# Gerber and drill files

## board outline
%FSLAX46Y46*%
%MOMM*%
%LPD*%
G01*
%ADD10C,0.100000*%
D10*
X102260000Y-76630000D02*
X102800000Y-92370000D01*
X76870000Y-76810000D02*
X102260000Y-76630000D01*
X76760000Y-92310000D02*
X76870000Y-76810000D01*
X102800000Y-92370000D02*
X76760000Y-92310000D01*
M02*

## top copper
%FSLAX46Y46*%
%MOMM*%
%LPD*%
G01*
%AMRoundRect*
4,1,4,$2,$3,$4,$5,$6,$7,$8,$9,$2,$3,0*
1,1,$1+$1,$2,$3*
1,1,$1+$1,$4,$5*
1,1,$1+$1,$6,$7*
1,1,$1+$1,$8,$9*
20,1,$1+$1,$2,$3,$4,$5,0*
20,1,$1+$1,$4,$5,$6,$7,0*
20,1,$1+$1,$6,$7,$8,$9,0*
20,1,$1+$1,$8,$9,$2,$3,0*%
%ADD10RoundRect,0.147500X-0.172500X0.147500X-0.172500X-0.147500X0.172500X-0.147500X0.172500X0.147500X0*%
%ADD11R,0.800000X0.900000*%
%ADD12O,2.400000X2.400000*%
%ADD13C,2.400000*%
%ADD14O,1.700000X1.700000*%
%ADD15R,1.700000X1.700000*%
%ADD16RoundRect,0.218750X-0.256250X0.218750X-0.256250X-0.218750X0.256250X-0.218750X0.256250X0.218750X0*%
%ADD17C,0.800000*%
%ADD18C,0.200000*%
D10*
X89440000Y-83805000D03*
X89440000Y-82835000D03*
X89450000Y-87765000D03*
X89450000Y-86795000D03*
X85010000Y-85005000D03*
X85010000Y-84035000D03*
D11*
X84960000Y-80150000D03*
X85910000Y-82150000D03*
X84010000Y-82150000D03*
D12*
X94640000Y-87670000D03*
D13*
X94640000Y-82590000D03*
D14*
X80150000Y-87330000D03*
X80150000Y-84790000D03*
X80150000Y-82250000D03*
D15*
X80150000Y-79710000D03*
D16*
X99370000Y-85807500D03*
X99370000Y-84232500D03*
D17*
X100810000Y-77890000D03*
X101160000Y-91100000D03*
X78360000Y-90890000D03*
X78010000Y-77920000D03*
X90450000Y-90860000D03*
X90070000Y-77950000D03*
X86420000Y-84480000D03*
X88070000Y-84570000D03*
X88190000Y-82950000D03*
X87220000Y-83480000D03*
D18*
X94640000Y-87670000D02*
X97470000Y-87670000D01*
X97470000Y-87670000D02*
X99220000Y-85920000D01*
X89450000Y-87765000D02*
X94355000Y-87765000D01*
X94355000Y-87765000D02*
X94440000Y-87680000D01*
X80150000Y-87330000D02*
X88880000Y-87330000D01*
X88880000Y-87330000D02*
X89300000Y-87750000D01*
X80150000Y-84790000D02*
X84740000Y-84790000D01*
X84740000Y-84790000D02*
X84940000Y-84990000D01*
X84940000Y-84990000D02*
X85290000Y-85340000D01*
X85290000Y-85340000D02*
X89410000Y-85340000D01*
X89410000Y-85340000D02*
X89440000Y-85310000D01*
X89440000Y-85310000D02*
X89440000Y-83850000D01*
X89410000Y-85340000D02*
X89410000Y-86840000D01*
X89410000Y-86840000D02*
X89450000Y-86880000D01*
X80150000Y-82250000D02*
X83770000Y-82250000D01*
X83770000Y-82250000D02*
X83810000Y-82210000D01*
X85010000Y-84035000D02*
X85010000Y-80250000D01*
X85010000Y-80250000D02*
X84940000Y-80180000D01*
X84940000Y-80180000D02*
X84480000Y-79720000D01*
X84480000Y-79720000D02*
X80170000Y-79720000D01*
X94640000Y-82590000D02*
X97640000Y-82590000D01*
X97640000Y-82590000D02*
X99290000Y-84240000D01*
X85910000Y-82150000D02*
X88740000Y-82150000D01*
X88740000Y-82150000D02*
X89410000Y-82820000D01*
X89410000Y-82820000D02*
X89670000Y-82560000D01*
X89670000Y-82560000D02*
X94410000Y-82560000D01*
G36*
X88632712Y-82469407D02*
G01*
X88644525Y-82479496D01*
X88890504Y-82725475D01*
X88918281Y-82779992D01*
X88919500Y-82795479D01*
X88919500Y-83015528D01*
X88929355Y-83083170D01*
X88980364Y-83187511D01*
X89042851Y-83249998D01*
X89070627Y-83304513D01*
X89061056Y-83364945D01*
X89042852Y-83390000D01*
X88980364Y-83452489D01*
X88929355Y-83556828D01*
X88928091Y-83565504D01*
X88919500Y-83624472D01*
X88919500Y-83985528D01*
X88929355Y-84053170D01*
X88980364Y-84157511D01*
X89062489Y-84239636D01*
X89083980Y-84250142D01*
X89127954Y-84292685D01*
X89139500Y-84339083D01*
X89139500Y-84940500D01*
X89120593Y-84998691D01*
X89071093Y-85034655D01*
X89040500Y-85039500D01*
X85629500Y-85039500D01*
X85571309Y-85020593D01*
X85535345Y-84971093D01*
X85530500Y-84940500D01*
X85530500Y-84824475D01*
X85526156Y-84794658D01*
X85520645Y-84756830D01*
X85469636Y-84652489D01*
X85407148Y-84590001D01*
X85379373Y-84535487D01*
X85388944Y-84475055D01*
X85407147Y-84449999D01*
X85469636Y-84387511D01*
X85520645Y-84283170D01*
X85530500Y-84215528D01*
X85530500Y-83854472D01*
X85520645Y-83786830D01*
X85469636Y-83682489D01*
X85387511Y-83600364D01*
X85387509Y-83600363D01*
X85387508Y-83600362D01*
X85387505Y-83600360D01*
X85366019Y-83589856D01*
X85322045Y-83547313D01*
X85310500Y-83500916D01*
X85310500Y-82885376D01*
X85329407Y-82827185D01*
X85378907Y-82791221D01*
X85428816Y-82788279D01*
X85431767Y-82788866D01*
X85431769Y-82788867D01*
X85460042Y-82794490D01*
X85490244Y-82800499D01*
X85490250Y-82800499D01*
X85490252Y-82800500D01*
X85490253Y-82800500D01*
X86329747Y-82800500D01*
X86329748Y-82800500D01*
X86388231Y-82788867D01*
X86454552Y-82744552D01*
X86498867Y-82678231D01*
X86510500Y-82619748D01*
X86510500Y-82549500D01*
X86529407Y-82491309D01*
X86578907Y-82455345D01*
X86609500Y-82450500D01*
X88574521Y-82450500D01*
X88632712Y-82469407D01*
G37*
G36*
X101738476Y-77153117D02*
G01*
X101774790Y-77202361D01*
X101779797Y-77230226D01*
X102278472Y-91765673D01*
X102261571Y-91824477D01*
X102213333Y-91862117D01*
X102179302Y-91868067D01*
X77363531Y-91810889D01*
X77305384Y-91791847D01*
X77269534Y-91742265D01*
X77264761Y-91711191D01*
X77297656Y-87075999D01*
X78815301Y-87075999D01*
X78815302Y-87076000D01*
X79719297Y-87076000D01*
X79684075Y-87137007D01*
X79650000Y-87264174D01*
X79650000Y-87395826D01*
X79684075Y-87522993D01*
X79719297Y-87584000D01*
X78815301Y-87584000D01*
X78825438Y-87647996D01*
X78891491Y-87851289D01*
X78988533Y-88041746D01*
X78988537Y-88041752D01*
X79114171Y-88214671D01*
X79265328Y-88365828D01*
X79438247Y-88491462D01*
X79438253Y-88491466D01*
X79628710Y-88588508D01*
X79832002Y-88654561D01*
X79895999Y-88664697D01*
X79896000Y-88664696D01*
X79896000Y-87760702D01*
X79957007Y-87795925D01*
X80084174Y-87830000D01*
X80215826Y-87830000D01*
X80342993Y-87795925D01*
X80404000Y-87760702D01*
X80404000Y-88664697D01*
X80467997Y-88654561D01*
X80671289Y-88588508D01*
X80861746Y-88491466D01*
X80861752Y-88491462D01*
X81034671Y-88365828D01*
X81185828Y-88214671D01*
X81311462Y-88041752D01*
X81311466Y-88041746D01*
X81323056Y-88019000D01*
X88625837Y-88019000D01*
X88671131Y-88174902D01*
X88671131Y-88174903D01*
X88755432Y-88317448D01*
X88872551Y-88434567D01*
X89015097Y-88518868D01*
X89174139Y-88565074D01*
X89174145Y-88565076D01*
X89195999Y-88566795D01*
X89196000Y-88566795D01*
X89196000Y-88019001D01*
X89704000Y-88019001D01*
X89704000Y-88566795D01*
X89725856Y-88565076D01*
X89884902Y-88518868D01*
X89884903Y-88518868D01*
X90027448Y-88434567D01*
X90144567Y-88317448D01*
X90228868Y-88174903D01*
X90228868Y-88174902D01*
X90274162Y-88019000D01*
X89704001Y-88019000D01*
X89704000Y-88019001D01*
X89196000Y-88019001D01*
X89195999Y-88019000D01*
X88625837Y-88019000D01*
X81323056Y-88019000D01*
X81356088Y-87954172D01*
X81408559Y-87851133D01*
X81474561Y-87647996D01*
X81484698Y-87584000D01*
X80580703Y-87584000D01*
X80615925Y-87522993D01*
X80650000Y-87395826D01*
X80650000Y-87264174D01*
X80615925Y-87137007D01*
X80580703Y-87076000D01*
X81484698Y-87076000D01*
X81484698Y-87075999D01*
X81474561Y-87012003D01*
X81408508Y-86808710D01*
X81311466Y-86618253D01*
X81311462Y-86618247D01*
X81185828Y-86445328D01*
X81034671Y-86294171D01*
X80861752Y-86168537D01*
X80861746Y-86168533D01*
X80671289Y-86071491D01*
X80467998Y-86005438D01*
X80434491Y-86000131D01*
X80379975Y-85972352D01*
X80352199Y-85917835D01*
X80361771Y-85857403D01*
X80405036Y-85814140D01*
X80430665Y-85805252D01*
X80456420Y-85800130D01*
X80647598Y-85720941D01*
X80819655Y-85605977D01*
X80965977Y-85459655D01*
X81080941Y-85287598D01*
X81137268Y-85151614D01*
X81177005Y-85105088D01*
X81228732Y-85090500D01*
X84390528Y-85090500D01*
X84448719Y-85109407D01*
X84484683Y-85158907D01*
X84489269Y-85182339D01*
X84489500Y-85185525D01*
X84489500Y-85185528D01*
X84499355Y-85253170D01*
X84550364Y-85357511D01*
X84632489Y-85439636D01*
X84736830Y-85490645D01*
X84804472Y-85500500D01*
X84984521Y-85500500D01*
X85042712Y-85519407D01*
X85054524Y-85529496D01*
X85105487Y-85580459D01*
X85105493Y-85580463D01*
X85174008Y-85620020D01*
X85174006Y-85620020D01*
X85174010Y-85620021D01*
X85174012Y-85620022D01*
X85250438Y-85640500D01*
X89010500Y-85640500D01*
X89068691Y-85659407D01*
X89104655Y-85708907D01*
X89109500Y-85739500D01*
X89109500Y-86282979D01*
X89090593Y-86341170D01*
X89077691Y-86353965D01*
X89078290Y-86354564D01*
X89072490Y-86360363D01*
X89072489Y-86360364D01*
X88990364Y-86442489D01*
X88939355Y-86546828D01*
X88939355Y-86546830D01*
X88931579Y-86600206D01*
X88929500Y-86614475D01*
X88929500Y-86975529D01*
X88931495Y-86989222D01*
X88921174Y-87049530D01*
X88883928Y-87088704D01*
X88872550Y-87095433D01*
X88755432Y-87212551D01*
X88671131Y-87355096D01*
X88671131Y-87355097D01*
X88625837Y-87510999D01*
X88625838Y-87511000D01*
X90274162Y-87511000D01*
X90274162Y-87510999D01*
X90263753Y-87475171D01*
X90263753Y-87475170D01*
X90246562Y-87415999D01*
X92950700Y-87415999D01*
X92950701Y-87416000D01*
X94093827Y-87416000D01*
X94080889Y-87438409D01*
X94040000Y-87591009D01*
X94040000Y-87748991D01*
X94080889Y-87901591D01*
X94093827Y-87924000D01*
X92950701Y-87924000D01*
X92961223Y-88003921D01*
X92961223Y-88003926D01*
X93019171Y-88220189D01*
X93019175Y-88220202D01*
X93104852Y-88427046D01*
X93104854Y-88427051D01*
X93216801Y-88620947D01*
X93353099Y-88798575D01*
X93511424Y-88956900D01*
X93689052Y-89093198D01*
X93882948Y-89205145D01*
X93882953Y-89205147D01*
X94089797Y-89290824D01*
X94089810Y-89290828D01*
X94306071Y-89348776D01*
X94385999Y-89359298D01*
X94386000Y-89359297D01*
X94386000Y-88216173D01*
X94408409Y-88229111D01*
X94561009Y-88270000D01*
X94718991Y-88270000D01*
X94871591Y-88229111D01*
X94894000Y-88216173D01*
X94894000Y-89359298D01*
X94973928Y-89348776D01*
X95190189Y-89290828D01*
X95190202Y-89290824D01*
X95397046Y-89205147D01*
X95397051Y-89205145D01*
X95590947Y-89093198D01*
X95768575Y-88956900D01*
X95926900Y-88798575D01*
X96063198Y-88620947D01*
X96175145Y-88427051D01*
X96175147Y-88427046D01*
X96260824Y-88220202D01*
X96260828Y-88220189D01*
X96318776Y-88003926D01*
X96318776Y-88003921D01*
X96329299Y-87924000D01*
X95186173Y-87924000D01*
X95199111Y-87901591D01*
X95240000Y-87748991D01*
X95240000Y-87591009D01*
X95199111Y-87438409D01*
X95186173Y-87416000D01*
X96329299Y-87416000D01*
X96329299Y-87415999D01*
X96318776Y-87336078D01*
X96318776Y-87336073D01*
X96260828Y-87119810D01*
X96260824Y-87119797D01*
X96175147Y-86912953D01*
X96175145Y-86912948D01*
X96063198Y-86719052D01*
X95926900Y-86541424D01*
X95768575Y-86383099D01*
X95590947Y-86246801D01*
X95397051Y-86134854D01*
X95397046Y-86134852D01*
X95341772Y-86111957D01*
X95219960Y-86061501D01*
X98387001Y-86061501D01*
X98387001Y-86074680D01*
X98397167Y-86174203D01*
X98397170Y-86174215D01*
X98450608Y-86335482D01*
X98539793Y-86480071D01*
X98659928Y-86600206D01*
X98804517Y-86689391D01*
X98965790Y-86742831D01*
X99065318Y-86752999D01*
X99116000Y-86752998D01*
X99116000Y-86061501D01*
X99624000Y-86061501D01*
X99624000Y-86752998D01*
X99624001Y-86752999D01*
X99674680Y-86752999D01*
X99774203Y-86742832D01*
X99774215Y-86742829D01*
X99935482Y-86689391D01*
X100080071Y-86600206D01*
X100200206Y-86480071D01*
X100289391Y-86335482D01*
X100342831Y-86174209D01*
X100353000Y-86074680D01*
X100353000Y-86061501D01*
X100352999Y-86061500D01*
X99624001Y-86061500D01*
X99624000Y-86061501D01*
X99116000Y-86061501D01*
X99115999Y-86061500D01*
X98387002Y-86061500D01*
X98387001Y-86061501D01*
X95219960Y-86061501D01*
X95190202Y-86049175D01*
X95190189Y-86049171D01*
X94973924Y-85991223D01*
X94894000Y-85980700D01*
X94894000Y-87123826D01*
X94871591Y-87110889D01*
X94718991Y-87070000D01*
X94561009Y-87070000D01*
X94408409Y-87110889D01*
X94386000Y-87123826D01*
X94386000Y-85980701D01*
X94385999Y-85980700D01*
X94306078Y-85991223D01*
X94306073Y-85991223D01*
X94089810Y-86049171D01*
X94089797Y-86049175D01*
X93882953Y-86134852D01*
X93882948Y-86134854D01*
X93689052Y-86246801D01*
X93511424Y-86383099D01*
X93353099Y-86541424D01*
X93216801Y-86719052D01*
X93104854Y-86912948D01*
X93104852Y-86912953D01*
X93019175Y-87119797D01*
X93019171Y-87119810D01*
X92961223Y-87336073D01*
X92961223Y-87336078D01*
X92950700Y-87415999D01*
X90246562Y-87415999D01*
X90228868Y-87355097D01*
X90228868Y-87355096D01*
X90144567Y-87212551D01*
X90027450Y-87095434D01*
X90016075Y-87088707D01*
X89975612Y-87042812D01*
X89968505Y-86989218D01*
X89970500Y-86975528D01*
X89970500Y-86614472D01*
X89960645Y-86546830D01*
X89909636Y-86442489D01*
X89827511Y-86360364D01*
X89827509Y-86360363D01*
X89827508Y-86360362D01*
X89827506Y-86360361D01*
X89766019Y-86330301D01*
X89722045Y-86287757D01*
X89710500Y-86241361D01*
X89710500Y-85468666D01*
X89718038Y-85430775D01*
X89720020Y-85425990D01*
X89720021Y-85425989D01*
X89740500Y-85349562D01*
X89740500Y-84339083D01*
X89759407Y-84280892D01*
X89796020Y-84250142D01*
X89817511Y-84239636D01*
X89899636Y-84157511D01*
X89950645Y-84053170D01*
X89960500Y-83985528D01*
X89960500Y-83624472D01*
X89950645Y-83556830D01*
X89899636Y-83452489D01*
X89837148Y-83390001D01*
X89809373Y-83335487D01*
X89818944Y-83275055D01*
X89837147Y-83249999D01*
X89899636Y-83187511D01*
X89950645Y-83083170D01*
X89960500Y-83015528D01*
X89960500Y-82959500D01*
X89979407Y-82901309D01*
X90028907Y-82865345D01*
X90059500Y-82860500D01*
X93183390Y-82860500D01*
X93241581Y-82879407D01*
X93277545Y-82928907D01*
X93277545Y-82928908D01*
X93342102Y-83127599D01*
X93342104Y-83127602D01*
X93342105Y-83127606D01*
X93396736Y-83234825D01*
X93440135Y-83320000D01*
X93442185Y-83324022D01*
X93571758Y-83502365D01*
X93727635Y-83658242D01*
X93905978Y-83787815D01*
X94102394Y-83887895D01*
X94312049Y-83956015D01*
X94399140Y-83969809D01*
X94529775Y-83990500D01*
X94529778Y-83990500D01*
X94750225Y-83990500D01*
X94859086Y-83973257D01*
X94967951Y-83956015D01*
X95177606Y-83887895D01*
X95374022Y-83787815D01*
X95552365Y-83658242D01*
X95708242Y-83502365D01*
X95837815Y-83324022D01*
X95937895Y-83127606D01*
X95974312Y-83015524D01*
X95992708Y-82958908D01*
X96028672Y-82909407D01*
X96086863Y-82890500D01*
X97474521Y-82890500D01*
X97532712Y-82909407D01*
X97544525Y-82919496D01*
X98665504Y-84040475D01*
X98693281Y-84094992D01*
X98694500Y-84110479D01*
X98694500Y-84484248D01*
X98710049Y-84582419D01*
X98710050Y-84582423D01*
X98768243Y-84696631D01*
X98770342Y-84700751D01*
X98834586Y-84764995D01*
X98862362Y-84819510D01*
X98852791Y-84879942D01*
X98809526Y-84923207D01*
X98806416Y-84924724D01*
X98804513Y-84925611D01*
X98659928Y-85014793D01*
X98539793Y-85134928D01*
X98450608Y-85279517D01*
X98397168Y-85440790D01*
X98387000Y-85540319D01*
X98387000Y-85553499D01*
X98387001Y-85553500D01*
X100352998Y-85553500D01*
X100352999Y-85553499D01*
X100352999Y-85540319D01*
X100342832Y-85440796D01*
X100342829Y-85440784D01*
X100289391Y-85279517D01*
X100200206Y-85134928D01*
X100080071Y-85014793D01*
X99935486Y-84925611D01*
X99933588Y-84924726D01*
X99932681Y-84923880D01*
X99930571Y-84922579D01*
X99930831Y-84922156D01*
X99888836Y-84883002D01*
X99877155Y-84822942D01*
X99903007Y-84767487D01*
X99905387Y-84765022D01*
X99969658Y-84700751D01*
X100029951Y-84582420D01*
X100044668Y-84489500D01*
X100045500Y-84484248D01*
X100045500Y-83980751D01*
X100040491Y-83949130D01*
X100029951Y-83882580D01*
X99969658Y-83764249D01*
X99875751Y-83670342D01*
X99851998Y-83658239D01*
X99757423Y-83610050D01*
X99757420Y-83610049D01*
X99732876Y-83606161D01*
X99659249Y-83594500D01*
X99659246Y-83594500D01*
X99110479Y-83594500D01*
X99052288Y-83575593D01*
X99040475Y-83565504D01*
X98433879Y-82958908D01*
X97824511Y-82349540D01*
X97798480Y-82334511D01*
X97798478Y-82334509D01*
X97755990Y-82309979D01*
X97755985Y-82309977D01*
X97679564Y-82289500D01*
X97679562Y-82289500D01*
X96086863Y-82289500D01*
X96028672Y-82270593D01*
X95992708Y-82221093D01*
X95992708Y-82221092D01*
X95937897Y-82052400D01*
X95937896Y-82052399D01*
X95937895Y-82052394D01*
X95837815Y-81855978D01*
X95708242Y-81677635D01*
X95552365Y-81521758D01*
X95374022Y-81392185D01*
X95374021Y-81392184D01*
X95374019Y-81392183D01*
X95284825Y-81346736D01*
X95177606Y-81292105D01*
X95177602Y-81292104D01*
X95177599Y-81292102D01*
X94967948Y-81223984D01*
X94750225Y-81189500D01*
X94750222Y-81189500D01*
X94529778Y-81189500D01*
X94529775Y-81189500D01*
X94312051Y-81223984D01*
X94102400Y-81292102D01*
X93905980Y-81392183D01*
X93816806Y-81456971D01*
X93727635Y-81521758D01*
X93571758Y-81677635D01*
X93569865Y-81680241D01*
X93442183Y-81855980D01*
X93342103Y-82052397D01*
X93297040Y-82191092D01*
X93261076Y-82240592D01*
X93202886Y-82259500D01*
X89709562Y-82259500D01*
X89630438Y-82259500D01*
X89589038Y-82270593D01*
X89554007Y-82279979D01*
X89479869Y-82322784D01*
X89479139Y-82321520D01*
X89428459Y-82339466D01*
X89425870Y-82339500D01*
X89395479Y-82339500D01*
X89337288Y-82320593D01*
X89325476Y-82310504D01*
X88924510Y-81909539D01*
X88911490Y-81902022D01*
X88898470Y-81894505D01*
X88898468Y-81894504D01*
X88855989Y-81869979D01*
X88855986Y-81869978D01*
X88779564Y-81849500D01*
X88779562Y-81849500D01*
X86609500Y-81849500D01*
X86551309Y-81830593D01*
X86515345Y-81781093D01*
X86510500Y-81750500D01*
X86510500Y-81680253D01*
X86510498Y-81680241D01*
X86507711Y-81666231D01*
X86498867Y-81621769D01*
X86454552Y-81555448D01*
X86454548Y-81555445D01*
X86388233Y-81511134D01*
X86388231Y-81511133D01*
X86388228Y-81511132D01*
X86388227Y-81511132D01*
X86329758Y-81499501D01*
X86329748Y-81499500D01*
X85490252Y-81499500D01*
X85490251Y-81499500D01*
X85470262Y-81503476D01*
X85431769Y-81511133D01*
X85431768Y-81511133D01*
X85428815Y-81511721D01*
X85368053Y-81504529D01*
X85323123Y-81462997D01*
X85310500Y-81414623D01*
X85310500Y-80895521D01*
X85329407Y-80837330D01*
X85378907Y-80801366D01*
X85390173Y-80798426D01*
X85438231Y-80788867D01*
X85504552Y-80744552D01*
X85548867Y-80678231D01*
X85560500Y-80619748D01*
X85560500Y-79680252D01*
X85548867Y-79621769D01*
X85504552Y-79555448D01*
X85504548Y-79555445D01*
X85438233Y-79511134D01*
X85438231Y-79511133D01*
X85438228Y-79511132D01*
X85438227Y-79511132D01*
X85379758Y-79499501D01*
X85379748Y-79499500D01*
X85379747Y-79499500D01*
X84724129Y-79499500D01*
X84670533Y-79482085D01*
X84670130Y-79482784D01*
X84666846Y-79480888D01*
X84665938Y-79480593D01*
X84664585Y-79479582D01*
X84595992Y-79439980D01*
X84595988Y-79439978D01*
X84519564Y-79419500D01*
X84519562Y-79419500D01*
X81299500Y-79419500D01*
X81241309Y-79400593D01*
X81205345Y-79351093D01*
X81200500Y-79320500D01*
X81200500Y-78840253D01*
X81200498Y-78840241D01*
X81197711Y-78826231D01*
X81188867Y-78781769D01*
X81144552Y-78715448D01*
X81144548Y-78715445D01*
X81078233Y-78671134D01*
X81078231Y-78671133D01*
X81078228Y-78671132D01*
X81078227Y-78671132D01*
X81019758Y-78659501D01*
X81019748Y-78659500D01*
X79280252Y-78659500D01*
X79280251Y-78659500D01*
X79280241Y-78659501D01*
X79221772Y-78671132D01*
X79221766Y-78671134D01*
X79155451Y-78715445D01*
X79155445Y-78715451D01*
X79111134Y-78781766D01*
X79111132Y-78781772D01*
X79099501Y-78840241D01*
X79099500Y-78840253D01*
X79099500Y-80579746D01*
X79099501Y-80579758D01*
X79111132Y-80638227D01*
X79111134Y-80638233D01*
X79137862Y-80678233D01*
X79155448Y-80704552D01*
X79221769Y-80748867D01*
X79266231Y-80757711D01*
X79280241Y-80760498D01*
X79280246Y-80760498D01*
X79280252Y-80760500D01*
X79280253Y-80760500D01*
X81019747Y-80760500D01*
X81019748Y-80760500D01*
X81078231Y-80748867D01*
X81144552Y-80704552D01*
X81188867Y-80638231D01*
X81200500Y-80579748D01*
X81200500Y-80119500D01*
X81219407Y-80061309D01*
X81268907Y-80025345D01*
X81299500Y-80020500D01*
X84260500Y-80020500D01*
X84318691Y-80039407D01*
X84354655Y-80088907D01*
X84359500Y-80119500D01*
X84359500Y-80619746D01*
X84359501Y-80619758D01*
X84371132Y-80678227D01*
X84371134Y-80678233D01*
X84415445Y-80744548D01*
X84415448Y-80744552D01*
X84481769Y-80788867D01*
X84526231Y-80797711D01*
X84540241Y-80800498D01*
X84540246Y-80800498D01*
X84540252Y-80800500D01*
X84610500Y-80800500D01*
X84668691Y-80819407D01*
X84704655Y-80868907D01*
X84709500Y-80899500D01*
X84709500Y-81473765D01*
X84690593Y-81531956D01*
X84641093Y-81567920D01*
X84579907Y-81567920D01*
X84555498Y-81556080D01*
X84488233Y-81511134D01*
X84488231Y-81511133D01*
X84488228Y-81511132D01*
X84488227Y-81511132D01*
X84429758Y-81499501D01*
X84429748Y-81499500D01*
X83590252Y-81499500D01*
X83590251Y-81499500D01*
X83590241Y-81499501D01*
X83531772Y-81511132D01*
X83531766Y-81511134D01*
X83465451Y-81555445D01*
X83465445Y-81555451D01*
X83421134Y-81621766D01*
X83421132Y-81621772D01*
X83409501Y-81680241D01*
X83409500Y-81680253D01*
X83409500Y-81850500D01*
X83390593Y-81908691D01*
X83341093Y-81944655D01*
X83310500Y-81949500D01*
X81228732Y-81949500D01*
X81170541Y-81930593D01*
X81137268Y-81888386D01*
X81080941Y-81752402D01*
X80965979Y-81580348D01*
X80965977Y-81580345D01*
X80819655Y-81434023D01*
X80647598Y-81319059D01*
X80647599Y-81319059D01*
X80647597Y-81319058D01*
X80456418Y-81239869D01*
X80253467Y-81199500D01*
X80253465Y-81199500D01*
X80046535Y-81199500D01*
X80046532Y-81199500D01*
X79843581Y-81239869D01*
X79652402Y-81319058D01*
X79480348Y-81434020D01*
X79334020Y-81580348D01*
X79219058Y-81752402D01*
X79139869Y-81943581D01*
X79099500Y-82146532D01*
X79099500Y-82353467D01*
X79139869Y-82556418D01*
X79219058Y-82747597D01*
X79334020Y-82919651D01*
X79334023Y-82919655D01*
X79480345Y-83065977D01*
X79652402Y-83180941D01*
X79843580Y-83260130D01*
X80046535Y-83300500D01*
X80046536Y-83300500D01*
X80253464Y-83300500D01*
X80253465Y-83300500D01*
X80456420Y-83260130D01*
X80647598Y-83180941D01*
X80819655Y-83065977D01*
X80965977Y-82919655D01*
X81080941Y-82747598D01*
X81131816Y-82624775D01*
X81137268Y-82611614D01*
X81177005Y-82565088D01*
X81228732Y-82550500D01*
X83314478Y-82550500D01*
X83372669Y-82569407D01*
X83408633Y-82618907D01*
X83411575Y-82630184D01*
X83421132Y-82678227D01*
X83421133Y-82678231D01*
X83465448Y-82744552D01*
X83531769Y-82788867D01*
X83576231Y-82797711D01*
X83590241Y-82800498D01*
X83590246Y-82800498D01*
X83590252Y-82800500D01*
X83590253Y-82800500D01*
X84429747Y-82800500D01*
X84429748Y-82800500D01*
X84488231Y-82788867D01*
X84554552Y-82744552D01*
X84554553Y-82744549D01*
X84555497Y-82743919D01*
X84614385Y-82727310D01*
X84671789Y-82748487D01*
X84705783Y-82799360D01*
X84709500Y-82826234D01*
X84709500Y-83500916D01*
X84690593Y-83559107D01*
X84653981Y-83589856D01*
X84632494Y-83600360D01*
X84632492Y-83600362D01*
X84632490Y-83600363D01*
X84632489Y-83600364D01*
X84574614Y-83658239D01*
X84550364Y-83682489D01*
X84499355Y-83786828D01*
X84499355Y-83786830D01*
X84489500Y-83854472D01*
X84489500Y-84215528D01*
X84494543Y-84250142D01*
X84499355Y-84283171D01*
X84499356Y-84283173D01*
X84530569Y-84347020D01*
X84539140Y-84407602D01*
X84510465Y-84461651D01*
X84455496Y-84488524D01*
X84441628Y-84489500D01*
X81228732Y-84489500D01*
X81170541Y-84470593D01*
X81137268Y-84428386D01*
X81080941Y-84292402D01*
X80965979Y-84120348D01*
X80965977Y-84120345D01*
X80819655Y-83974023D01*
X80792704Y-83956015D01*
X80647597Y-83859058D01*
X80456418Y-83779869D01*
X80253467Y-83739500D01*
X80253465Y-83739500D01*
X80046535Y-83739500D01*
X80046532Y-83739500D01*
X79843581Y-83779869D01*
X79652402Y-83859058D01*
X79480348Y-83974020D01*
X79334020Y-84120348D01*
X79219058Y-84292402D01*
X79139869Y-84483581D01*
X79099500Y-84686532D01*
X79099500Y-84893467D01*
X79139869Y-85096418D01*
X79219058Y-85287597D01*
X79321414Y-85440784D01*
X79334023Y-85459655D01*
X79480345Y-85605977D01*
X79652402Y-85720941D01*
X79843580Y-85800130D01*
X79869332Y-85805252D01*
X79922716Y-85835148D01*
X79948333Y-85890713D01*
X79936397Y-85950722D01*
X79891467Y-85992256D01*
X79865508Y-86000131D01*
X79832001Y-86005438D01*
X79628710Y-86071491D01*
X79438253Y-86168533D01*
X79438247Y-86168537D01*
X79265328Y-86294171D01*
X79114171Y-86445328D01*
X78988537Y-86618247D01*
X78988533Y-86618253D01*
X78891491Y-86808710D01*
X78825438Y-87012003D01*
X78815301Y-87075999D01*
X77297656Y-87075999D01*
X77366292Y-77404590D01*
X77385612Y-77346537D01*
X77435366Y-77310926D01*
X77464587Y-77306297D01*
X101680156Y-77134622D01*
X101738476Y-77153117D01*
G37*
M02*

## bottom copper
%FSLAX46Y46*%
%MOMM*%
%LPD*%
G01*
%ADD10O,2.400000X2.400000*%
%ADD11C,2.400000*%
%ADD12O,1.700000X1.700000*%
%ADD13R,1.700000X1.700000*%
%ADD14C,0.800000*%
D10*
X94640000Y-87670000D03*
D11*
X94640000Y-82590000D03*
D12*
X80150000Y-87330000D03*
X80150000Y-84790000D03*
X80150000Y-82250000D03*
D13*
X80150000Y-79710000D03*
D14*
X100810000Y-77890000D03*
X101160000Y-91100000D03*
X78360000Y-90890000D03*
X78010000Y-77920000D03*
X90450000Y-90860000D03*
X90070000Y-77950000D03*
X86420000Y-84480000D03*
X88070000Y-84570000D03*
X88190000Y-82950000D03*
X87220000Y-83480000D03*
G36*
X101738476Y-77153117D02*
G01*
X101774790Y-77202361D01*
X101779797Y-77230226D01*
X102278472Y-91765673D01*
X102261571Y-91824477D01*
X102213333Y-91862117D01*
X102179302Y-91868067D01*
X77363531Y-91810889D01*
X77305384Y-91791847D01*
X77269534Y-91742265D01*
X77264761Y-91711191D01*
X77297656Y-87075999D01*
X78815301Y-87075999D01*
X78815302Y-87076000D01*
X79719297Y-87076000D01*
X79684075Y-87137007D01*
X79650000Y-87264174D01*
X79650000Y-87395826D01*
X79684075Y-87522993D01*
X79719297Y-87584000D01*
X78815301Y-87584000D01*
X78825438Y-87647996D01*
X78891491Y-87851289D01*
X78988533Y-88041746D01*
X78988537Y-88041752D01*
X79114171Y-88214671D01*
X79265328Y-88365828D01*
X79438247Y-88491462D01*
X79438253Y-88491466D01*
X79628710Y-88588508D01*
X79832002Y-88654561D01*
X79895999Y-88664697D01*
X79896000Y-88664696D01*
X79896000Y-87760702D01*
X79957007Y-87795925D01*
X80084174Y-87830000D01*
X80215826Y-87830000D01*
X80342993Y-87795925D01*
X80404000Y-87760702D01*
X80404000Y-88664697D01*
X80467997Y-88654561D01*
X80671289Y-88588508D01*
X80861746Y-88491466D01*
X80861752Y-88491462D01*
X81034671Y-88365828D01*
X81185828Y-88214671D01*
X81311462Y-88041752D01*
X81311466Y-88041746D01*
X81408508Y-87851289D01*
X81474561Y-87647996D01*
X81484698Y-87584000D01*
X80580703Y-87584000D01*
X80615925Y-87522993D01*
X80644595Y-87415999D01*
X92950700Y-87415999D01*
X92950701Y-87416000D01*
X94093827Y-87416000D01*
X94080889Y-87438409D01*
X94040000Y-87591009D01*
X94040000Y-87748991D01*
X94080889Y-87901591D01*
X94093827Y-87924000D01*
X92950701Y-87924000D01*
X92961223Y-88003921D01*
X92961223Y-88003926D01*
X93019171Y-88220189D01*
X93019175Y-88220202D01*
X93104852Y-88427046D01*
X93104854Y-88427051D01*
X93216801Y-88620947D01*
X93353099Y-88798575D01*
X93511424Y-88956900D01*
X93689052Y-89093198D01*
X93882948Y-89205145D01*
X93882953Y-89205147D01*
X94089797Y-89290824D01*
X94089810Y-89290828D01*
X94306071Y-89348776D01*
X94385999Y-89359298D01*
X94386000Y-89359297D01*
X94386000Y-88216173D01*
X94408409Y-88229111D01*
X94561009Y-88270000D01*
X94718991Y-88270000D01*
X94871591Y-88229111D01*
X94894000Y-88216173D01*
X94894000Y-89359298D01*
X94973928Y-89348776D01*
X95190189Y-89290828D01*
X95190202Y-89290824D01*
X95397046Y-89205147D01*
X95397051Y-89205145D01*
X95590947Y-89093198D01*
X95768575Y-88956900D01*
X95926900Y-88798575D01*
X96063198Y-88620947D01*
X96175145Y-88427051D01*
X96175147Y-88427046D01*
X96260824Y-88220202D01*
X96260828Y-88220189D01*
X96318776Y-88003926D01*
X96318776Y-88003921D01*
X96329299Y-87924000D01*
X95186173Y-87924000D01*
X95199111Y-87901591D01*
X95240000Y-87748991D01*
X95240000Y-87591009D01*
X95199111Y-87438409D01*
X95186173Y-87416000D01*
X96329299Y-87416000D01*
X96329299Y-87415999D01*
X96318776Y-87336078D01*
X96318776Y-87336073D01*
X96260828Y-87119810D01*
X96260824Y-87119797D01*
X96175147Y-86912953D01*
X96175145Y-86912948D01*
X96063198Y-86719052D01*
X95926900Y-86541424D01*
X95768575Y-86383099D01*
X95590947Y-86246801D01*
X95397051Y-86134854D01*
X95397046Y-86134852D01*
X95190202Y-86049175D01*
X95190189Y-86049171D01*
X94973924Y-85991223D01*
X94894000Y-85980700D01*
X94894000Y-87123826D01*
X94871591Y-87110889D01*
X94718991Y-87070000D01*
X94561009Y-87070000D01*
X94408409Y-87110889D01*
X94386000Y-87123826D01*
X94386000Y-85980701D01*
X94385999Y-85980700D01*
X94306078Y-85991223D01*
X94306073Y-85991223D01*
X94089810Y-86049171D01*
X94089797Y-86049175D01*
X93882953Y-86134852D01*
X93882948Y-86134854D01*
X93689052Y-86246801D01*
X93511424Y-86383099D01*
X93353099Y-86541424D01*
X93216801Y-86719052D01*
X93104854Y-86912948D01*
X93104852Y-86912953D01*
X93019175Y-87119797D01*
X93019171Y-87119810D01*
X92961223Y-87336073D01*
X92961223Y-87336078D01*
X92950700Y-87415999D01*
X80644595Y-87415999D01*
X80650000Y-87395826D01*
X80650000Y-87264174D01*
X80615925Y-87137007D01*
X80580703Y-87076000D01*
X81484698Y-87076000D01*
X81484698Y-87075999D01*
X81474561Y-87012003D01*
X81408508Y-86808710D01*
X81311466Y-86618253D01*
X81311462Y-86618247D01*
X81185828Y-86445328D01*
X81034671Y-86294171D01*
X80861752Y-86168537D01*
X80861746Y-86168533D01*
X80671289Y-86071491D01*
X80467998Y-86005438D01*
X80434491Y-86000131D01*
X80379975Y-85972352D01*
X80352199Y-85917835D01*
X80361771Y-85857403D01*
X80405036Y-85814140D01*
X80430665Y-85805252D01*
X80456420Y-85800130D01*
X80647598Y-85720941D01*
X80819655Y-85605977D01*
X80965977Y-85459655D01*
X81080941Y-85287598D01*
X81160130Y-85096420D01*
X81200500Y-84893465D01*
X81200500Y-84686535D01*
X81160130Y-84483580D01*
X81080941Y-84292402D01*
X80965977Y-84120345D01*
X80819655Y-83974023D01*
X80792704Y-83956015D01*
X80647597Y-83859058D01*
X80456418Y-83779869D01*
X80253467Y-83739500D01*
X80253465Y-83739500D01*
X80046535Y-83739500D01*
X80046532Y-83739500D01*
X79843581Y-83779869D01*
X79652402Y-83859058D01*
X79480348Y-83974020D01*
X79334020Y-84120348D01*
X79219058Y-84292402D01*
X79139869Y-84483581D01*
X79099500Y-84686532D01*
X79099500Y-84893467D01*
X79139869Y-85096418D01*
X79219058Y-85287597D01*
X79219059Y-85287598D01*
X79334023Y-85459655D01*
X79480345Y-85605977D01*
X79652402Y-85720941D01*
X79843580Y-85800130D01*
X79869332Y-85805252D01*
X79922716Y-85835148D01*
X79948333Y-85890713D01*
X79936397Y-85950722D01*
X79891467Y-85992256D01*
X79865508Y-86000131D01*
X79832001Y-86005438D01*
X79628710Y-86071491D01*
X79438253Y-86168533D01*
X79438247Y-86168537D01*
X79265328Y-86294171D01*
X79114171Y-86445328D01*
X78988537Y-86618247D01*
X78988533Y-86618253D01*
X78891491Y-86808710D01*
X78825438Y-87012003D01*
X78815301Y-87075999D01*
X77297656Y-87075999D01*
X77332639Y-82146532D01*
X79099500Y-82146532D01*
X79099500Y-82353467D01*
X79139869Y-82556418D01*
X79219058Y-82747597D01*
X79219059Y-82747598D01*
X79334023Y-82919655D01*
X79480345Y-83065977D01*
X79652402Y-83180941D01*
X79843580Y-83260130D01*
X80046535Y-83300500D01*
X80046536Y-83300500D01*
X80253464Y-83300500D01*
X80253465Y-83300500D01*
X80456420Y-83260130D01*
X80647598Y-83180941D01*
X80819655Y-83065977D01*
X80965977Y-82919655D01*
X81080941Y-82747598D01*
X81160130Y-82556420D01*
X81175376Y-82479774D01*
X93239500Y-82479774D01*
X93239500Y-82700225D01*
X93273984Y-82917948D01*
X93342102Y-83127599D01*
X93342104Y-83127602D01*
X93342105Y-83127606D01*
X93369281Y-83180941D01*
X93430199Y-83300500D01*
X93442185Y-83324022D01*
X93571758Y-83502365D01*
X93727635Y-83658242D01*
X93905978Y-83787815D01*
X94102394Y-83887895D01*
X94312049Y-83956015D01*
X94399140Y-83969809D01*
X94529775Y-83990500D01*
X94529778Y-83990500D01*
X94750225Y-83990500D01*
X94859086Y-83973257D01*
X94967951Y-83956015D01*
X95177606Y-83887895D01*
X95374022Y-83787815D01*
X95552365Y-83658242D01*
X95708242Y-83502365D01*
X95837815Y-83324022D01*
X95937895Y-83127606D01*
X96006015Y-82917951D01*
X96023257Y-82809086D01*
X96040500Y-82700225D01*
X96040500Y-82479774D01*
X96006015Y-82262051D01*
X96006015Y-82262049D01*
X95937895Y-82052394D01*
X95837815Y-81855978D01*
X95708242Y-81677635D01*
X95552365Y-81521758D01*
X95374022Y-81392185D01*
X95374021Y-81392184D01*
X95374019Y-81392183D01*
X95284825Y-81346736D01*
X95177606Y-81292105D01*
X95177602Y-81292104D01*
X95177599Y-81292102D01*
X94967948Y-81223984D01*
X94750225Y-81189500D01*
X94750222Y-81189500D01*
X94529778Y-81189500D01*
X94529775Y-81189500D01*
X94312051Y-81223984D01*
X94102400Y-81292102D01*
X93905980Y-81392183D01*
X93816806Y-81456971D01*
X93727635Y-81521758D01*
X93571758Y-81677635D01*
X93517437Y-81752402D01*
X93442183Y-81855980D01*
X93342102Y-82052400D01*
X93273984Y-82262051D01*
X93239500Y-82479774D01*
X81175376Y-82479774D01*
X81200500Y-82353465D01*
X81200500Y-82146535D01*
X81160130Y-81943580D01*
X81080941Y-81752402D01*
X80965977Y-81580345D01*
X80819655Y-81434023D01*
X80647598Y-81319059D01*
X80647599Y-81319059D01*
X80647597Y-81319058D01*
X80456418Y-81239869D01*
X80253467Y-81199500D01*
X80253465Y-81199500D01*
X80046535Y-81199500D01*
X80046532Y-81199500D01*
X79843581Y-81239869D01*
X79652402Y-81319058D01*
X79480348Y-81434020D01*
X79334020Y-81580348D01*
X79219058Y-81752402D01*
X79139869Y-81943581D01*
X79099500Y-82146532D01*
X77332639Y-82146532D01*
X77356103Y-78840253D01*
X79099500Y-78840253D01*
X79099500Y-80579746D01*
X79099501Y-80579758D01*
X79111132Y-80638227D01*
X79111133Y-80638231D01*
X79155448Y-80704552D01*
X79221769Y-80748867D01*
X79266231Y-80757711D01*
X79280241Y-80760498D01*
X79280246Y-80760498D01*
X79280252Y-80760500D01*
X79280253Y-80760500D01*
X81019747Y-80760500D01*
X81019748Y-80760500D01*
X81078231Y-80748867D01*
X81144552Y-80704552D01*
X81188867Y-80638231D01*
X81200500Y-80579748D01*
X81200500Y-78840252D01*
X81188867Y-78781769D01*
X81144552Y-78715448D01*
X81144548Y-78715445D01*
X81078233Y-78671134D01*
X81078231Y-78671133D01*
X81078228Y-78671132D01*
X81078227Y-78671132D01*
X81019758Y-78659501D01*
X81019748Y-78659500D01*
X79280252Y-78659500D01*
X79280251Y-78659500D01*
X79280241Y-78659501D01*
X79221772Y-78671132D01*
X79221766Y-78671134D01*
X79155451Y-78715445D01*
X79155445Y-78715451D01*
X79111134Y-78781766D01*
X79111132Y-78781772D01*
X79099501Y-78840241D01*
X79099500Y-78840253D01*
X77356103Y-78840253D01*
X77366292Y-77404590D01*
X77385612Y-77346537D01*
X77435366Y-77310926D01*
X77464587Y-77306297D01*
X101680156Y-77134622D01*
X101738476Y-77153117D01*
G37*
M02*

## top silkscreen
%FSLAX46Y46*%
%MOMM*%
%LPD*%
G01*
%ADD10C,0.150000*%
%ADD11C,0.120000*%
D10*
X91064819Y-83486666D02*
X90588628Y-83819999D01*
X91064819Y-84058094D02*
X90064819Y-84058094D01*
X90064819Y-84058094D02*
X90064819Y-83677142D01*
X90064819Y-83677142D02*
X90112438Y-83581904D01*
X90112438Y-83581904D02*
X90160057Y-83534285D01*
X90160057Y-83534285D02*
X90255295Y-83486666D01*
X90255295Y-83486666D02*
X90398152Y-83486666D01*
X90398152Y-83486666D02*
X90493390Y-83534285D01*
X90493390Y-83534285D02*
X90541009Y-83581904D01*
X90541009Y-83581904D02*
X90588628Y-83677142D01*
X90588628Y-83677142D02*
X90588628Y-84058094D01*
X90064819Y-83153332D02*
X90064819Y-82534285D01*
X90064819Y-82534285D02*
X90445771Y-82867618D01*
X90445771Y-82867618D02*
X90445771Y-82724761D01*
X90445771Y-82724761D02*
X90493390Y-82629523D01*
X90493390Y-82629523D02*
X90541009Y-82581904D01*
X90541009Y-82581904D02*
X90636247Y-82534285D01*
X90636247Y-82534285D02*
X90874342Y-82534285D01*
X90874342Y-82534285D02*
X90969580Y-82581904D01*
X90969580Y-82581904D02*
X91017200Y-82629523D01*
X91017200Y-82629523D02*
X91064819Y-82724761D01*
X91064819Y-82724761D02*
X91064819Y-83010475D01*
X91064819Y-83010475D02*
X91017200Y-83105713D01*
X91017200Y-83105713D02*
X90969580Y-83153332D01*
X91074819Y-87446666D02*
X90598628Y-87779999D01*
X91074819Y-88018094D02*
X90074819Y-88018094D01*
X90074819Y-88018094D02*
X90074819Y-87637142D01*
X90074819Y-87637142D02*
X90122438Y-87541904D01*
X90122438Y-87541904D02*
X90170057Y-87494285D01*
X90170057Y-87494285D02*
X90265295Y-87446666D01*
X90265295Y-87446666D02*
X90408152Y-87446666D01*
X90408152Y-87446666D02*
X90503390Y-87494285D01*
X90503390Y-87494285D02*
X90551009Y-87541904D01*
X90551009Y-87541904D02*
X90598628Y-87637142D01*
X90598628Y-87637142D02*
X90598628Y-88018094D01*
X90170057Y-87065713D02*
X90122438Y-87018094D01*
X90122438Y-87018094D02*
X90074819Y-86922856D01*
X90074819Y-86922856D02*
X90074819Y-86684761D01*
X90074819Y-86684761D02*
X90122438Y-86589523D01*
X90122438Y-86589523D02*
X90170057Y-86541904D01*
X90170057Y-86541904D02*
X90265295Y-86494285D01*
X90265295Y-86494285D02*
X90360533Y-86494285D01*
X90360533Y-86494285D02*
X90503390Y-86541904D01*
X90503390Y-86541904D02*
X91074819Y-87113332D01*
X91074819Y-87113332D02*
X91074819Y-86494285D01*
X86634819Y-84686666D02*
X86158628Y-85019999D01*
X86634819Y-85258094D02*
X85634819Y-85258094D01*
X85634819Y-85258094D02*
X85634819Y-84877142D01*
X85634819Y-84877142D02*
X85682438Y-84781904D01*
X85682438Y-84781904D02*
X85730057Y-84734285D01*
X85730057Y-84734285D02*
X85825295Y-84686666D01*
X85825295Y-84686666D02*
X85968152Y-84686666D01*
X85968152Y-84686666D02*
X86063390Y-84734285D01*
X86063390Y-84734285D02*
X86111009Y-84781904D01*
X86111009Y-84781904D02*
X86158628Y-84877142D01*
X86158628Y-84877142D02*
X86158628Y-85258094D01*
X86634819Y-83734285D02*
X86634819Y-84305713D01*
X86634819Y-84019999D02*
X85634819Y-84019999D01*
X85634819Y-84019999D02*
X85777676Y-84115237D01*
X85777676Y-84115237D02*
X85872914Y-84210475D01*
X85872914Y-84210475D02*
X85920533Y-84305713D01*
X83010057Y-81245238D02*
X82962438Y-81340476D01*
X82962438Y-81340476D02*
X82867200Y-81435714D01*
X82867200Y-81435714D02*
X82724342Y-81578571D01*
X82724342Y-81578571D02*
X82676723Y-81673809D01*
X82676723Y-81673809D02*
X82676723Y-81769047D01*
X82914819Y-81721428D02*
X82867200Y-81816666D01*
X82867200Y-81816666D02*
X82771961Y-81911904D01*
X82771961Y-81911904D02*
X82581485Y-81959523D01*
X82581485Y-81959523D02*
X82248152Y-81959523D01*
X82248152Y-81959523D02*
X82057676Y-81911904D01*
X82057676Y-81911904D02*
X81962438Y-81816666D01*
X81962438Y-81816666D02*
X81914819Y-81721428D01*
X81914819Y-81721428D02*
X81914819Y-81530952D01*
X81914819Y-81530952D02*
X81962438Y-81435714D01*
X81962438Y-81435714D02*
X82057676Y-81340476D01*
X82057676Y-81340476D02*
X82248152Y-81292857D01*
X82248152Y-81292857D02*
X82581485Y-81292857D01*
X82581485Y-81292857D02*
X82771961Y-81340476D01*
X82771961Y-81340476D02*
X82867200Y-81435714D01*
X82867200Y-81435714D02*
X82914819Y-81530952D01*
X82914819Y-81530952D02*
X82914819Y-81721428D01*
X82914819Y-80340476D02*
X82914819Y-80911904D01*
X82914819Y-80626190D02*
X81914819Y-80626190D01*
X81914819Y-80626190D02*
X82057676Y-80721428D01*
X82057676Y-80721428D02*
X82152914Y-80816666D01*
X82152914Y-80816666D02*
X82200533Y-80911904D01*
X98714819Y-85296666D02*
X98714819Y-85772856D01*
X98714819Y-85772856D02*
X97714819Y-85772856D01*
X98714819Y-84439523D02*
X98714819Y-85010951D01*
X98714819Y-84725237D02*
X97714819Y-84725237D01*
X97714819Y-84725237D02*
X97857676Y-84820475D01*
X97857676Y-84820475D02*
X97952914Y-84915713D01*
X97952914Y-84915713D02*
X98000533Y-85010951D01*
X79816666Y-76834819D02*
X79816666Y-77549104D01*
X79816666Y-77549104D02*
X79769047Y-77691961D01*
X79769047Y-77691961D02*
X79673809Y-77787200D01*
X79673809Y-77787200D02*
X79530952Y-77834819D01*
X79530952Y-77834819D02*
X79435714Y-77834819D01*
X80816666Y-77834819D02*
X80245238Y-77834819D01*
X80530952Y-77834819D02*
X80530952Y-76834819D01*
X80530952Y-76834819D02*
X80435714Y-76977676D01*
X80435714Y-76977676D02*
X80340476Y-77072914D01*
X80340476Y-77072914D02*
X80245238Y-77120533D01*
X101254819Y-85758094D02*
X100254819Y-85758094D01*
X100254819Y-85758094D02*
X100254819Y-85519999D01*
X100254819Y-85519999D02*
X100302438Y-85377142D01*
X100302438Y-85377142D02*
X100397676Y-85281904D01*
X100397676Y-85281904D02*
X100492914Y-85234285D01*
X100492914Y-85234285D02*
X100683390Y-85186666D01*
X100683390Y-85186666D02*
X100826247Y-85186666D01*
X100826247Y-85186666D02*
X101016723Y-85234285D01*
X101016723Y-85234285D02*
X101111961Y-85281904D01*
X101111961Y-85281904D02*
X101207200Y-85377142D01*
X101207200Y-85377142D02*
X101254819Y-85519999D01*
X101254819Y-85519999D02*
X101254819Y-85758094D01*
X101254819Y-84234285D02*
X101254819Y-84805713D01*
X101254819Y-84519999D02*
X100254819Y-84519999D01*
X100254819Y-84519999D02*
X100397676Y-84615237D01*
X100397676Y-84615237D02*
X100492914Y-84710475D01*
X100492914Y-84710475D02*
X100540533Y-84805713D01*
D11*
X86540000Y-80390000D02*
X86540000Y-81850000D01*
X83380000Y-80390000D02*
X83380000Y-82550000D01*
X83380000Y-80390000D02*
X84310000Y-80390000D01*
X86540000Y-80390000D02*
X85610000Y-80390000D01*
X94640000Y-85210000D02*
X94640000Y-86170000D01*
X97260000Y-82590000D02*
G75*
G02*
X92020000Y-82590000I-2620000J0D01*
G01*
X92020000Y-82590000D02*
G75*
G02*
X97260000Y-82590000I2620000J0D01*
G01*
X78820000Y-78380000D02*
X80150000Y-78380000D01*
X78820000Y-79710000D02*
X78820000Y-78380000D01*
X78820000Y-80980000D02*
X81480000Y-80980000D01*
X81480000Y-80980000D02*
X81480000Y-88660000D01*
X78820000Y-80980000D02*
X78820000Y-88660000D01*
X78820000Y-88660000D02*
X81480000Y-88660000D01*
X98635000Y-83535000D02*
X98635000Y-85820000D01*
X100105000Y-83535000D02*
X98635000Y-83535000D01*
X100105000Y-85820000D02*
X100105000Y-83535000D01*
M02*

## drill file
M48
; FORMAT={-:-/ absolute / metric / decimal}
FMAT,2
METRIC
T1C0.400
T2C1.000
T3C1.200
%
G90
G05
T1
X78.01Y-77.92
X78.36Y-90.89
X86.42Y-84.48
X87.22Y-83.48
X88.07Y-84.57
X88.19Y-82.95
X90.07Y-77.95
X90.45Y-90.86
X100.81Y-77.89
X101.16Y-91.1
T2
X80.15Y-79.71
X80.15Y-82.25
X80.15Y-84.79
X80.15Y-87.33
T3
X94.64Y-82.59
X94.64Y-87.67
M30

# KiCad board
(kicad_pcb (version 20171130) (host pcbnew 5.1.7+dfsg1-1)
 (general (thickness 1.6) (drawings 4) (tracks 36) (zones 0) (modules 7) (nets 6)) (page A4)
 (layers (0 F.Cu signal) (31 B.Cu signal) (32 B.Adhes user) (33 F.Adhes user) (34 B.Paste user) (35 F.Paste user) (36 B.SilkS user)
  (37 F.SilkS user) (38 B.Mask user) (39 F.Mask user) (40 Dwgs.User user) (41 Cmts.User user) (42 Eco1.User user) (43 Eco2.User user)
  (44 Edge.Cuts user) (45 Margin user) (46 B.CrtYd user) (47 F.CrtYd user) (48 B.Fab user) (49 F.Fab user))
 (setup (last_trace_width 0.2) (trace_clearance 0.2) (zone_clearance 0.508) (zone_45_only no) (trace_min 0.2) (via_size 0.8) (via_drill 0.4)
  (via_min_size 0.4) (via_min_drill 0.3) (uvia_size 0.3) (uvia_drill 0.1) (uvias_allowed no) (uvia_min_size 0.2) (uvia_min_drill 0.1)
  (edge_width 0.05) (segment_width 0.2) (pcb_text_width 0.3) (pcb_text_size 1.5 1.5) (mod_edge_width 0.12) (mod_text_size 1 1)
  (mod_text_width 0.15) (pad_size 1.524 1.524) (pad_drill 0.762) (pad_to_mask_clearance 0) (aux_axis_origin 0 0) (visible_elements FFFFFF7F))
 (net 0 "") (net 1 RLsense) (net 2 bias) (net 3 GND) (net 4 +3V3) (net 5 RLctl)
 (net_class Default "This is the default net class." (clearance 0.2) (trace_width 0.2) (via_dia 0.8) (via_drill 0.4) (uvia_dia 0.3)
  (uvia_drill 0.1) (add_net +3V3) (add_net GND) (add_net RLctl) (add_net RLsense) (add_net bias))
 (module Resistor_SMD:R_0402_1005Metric (layer F.Cu) (at 89.44 83.32 270)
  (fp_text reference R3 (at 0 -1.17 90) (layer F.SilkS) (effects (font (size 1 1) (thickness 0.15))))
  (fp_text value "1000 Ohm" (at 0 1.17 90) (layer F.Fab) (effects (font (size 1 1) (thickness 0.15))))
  (pad 2 smd roundrect (at 0.485 0 270) (size 0.59 0.64) (layers F.Cu F.Paste F.Mask) (roundrect_rratio 0.25) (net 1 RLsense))
  (pad 1 smd roundrect (at -0.485 0 270) (size 0.59 0.64) (layers F.Cu F.Paste F.Mask) (roundrect_rratio 0.25) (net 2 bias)))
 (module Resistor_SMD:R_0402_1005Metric (layer F.Cu) (at 89.45 87.28 270)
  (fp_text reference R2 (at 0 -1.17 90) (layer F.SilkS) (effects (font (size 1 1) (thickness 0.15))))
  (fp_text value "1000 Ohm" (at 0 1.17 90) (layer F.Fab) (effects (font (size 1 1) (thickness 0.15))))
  (pad 2 smd roundrect (at 0.485 0 270) (size 0.59 0.64) (layers F.Cu F.Paste F.Mask) (roundrect_rratio 0.25) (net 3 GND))
  (pad 1 smd roundrect (at -0.485 0 270) (size 0.59 0.64) (layers F.Cu F.Paste F.Mask) (roundrect_rratio 0.25) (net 1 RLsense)))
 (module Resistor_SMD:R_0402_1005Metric (layer F.Cu) (at 85.01 84.52 270)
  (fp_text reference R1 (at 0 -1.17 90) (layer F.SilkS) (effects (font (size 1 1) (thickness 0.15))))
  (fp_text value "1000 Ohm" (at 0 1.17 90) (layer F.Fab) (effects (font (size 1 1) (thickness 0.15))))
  (pad 2 smd roundrect (at 0.485 0 270) (size 0.59 0.64) (layers F.Cu F.Paste F.Mask) (roundrect_rratio 0.25) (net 1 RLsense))
  (pad 1 smd roundrect (at -0.485 0 270) (size 0.59 0.64) (layers F.Cu F.Paste F.Mask) (roundrect_rratio 0.25) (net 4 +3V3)))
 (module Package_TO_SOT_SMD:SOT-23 (layer F.Cu) (at 84.96 81.15 90)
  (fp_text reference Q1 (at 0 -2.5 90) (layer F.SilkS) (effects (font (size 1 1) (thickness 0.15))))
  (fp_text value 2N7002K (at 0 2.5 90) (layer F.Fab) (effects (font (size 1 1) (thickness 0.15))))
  (fp_line (start 0.76 1.58) (end -0.7 1.58) (layer F.SilkS) (width 0.12))
  (fp_line (start 0.76 -1.58) (end -1.4 -1.58) (layer F.SilkS) (width 0.12))
  (fp_line (start 0.76 -1.58) (end 0.76 -0.65) (layer F.SilkS) (width 0.12))
  (fp_line (start 0.76 1.58) (end 0.76 0.65) (layer F.SilkS) (width 0.12))
  (pad 3 smd rect (at 1 0 90) (size 0.9 0.8) (layers F.Cu F.Paste F.Mask) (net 4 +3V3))
  (pad 2 smd rect (at -1 0.95 90) (size 0.9 0.8) (layers F.Cu F.Paste F.Mask) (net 2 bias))
  (pad 1 smd rect (at -1 -0.95 90) (size 0.9 0.8) (layers F.Cu F.Paste F.Mask) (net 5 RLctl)))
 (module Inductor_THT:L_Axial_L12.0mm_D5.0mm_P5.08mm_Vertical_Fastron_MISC (layer F.Cu) (at 94.64 82.59 270)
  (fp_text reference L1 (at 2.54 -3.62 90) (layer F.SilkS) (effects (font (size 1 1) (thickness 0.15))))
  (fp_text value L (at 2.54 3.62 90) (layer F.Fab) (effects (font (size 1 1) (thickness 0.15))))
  (fp_line (start 2.62 0) (end 3.58 0) (layer F.SilkS) (width 0.12))
  (fp_circle (center 0 0) (end 2.62 0) (layer F.SilkS) (width 0.12))
  (pad 2 thru_hole oval (at 5.08 0 270) (size 2.4 2.4) (drill 1.2) (layers *.Cu *.Mask) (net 3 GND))
  (pad 1 thru_hole circle (at 0 0 270) (size 2.4 2.4) (drill 1.2) (layers *.Cu *.Mask) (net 2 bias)))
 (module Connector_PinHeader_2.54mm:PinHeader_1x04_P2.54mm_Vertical (layer F.Cu) (at 80.15 79.71)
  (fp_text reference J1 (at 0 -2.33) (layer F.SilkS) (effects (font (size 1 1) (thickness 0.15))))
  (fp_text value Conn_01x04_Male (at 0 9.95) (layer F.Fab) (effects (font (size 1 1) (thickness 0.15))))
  (fp_line (start -1.33 -1.33) (end 0 -1.33) (layer F.SilkS) (width 0.12))
  (fp_line (start -1.33 0) (end -1.33 -1.33) (layer F.SilkS) (width 0.12))
  (fp_line (start -1.33 1.27) (end 1.33 1.27) (layer F.SilkS) (width 0.12))
  (fp_line (start 1.33 1.27) (end 1.33 8.95) (layer F.SilkS) (width 0.12))
  (fp_line (start -1.33 1.27) (end -1.33 8.95) (layer F.SilkS) (width 0.12))
  (fp_line (start -1.33 8.95) (end 1.33 8.95) (layer F.SilkS) (width 0.12))
  (pad 4 thru_hole oval (at 0 7.62) (size 1.7 1.7) (drill 1) (layers *.Cu *.Mask) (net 3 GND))
  (pad 3 thru_hole oval (at 0 5.08) (size 1.7 1.7) (drill 1) (layers *.Cu *.Mask) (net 1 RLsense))
  (pad 2 thru_hole oval (at 0 2.54) (size 1.7 1.7) (drill 1) (layers *.Cu *.Mask) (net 5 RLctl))
  (pad 1 thru_hole rect (at 0 0) (size 1.7 1.7) (drill 1) (layers *.Cu *.Mask) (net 4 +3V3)))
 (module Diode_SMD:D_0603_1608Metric (layer F.Cu) (at 99.37 85.02 270)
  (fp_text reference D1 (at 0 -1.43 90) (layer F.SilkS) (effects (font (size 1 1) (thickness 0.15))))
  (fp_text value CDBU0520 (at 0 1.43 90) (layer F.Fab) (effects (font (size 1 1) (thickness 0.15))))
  (fp_line (start -1.485 0.735) (end 0.8 0.735) (layer F.SilkS) (width 0.12))
  (fp_line (start -1.485 -0.735) (end -1.485 0.735) (layer F.SilkS) (width 0.12))
  (fp_line (start 0.8 -0.735) (end -1.485 -0.735) (layer F.SilkS) (width 0.12))
  (pad 2 smd roundrect (at 0.7875 0 270) (size 0.875 0.95) (layers F.Cu F.Paste F.Mask) (roundrect_rratio 0.25) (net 3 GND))
  (pad 1 smd roundrect (at -0.7875 0 270) (size 0.875 0.95) (layers F.Cu F.Paste F.Mask) (roundrect_rratio 0.25) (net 2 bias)))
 (gr_line (start 102.26 76.63) (end 102.8 92.37) (layer Edge.Cuts) (width 0.1))
 (gr_line (start 76.87 76.81) (end 102.26 76.63) (layer Edge.Cuts) (width 0.1))
 (gr_line (start 76.76 92.31) (end 76.87 76.81) (layer Edge.Cuts) (width 0.1))
 (gr_line (start 102.8 92.37) (end 76.76 92.31) (layer Edge.Cuts) (width 0.1))
 (segment (start 94.64 87.67) (end 97.47 87.67) (width 0.2) (layer F.Cu) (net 3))
 (segment (start 97.47 87.67) (end 99.22 85.92) (width 0.2) (layer F.Cu) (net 3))
 (segment (start 89.45 87.765) (end 94.355 87.765) (width 0.2) (layer F.Cu) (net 3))
 (segment (start 94.355 87.765) (end 94.44 87.68) (width 0.2) (layer F.Cu) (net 3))
 (segment (start 80.15 87.33) (end 88.88 87.33) (width 0.2) (layer F.Cu) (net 3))
 (segment (start 88.88 87.33) (end 89.3 87.75) (width 0.2) (layer F.Cu) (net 3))
 (via (at 100.81 77.89) (size 0.8) (drill 0.4) (layers F.Cu B.Cu) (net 3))
 (via (at 101.16 91.1) (size 0.8) (drill 0.4) (layers F.Cu B.Cu) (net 3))
 (via (at 78.36 90.89) (size 0.8) (drill 0.4) (layers F.Cu B.Cu) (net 3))
 (via (at 78.01 77.92) (size 0.8) (drill 0.4) (layers F.Cu B.Cu) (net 3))
 (via (at 90.45 90.86) (size 0.8) (drill 0.4) (layers F.Cu B.Cu) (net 3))
 (via (at 90.07 77.95) (size 0.8) (drill 0.4) (layers F.Cu B.Cu) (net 3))
 (via (at 86.42 84.48) (size 0.8) (drill 0.4) (layers F.Cu B.Cu) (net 3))
 (via (at 88.07 84.57) (size 0.8) (drill 0.4) (layers F.Cu B.Cu) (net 3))
 (via (at 88.19 82.95) (size 0.8) (drill 0.4) (layers F.Cu B.Cu) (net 3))
 (via (at 87.22 83.48) (size 0.8) (drill 0.4) (layers F.Cu B.Cu) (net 3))
 (segment (start 80.15 84.79) (end 84.74 84.79) (width 0.2) (layer F.Cu) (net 1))
 (segment (start 84.74 84.79) (end 84.94 84.99) (width 0.2) (layer F.Cu) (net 1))
 (segment (start 84.94 84.99) (end 85.29 85.34) (width 0.2) (layer F.Cu) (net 1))
 (segment (start 85.29 85.34) (end 89.41 85.34) (width 0.2) (layer F.Cu) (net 1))
 (segment (start 89.41 85.34) (end 89.44 85.31) (width 0.2) (layer F.Cu) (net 1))
 (segment (start 89.44 85.31) (end 89.44 83.85) (width 0.2) (layer F.Cu) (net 1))
 (segment (start 89.41 85.34) (end 89.41 86.84) (width 0.2) (layer F.Cu) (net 1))
 (segment (start 89.41 86.84) (end 89.45 86.88) (width 0.2) (layer F.Cu) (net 1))
 (segment (start 80.15 82.25) (end 83.77 82.25) (width 0.2) (layer F.Cu) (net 5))
 (segment (start 83.77 82.25) (end 83.81 82.21) (width 0.2) (layer F.Cu) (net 5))
 (segment (start 85.01 84.035) (end 85.01 80.25) (width 0.2) (layer F.Cu) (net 4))
 (segment (start 85.01 80.25) (end 84.94 80.18) (width 0.2) (layer F.Cu) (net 4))
 (segment (start 84.94 80.18) (end 84.48 79.72) (width 0.2) (layer F.Cu) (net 4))
 (segment (start 84.48 79.72) (end 80.17 79.72) (width 0.2) (layer F.Cu) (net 4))
 (segment (start 94.64 82.59) (end 97.64 82.59) (width 0.2) (layer F.Cu) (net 2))
 (segment (start 97.64 82.59) (end 99.29 84.24) (width 0.2) (layer F.Cu) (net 2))
 (segment (start 85.91 82.15) (end 88.74 82.15) (width 0.2) (layer F.Cu) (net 2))
 (segment (start 88.74 82.15) (end 89.41 82.82) (width 0.2) (layer F.Cu) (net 2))
 (segment (start 89.41 82.82) (end 89.67 82.56) (width 0.2) (layer F.Cu) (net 2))
 (segment (start 89.67 82.56) (end 94.41 82.56) (width 0.2) (layer F.Cu) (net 2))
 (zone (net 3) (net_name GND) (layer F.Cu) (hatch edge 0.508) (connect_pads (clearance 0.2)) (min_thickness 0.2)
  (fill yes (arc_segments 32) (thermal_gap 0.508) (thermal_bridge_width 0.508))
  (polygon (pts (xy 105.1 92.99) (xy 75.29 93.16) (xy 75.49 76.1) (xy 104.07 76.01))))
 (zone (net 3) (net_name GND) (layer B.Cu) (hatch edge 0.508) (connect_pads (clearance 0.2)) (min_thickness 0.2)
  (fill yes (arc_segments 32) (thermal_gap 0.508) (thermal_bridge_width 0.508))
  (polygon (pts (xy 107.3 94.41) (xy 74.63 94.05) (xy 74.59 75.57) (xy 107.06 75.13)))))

